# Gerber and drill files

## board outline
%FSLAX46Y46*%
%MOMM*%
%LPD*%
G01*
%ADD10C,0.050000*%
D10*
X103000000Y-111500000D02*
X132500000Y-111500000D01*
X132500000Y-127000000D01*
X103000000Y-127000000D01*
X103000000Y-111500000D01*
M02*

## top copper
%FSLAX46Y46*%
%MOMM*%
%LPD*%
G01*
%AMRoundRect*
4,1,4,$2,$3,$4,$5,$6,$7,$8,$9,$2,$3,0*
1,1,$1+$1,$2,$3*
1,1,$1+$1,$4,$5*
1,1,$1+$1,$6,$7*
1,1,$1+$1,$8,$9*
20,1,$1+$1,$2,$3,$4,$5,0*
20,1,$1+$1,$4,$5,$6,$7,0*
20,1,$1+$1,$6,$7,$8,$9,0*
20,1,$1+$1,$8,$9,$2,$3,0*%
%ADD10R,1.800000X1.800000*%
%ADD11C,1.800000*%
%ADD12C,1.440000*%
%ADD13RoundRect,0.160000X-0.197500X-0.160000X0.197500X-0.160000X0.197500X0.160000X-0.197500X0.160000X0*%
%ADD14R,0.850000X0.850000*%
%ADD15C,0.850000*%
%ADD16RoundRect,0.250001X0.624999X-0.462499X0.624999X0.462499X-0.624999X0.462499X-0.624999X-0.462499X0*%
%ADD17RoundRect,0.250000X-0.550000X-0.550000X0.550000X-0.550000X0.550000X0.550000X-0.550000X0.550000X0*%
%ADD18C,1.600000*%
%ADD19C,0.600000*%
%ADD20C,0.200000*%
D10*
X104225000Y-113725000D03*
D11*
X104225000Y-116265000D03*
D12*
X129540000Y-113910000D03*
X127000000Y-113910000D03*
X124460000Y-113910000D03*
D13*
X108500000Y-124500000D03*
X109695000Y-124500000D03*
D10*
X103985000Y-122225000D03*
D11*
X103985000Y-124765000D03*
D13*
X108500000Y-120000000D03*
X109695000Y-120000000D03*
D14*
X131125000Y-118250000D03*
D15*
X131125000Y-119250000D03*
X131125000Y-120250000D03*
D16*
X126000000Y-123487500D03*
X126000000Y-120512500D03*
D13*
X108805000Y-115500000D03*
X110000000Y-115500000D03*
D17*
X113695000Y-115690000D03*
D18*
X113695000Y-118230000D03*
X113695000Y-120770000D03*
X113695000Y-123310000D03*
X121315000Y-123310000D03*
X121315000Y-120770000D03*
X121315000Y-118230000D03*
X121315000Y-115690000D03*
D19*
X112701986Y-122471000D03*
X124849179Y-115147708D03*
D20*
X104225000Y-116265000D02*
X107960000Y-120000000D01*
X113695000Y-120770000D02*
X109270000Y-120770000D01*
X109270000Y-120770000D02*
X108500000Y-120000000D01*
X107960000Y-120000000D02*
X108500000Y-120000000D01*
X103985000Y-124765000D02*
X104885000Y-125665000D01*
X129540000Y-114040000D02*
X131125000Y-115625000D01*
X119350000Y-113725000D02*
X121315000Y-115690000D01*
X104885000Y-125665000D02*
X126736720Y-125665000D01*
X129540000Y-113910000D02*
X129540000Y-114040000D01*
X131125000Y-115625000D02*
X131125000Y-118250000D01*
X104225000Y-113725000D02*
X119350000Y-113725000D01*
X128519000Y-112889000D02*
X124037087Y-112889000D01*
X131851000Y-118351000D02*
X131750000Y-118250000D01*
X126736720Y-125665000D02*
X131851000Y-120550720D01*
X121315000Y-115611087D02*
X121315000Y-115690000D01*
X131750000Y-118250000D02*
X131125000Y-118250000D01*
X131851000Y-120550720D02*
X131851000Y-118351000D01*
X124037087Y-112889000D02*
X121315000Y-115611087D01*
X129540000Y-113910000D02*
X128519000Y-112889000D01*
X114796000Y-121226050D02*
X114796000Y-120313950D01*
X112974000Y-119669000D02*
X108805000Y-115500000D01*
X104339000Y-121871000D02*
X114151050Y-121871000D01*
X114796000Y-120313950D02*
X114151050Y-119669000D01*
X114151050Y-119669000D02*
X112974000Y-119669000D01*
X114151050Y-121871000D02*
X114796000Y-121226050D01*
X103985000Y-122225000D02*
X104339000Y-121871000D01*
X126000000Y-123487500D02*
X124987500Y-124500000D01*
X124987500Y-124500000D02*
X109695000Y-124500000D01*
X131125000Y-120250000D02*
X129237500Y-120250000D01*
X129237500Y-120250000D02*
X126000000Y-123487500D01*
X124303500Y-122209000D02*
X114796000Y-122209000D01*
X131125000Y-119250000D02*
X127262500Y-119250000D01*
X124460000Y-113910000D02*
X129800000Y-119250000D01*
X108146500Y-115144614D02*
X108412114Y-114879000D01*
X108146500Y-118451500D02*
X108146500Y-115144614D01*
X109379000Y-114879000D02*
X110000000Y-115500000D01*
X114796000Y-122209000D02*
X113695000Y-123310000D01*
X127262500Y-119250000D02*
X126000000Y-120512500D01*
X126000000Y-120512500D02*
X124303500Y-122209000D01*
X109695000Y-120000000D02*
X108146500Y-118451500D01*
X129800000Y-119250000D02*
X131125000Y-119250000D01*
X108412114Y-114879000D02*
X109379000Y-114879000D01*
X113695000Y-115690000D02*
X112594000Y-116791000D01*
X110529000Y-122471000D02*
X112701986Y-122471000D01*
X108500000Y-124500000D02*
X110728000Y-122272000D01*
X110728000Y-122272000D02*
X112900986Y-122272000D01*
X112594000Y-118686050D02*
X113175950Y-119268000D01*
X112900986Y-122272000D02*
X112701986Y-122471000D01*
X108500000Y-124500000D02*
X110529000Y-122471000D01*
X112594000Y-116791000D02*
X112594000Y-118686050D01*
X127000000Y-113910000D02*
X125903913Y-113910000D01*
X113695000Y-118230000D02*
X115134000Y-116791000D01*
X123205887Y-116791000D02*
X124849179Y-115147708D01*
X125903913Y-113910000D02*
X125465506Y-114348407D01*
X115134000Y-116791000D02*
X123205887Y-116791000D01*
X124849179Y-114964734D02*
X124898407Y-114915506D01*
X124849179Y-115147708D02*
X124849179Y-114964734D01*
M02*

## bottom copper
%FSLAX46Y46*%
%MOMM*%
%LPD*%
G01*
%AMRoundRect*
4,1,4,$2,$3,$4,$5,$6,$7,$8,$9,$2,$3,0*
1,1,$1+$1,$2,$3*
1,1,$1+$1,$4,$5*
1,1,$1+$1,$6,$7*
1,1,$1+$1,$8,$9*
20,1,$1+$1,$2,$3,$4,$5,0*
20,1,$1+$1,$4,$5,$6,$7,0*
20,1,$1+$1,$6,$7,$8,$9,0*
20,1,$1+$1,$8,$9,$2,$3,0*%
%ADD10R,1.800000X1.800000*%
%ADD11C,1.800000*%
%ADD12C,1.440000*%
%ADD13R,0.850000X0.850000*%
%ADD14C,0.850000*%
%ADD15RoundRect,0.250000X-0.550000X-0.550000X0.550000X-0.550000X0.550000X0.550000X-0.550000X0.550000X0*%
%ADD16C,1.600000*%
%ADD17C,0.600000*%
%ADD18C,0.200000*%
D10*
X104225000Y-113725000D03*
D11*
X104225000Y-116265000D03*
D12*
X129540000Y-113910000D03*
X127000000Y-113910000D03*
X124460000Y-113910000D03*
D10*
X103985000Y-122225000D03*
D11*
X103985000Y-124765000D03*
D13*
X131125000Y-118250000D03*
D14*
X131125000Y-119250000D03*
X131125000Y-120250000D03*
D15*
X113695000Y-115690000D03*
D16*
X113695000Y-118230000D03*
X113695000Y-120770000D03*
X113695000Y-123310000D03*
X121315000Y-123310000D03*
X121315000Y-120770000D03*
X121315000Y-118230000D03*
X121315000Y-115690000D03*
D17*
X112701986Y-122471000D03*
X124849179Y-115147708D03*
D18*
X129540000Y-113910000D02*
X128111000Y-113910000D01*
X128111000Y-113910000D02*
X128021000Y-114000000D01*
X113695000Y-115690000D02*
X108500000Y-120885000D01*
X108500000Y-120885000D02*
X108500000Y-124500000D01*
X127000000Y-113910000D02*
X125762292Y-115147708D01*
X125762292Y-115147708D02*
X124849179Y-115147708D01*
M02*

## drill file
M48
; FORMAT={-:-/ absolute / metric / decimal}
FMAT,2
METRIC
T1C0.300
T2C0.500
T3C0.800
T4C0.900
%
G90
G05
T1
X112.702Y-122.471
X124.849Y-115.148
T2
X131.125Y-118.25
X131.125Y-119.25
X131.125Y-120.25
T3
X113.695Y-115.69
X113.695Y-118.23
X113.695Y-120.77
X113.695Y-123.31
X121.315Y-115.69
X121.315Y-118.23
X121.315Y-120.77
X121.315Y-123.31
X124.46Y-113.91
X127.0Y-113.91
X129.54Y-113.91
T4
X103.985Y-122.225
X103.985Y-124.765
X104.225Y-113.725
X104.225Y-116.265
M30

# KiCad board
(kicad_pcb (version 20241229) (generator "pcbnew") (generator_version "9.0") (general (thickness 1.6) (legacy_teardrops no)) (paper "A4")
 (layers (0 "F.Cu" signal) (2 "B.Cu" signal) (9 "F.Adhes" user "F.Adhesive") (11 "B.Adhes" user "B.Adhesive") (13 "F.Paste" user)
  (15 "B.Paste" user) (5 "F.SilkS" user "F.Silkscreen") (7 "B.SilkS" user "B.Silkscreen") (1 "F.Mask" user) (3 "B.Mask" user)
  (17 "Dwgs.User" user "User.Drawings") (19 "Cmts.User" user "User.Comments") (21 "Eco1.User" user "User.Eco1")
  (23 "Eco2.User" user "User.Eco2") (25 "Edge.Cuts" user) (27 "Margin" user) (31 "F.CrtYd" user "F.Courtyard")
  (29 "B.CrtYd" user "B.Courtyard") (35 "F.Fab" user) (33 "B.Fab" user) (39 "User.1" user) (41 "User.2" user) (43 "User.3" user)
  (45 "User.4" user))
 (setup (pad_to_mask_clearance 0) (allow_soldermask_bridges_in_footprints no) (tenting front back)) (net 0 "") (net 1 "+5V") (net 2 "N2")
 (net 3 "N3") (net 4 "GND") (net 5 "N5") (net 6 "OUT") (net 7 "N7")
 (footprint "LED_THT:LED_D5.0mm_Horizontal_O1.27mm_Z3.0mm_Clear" (layer "F.Cu") (at 104.225 113.725 -90)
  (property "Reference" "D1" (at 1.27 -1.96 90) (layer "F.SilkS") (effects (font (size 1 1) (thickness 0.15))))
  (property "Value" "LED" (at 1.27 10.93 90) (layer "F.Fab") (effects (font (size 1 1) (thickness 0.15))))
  (pad "1" thru_hole rect (at 0 0 270) (size 1.8 1.8) (drill 0.9) (layers "*.Cu" "*.Mask") (remove_unused_layers no) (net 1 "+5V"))
  (pad "2" thru_hole circle (at 2.54 0 270) (size 1.8 1.8) (drill 0.9) (layers "*.Cu" "*.Mask") (remove_unused_layers no) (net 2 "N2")))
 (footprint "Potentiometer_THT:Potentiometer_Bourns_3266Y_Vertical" (layer "F.Cu") (at 129.54 113.91)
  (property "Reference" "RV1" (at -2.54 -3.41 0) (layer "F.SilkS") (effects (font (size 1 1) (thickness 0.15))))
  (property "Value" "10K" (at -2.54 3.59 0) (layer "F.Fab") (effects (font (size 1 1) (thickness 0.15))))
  (pad "1" thru_hole circle (at 0 0) (size 1.44 1.44) (drill 0.8) (layers "*.Cu" "*.Mask") (remove_unused_layers no) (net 1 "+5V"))
  (pad "2" thru_hole circle (at -2.54 0) (size 1.44 1.44) (drill 0.8) (layers "*.Cu" "*.Mask") (remove_unused_layers no) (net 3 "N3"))
  (pad "3" thru_hole circle (at -5.08 0) (size 1.44 1.44) (drill 0.8) (layers "*.Cu" "*.Mask") (remove_unused_layers no) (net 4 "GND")))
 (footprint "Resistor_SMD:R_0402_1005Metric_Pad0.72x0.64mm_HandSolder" (layer "F.Cu") (at 109.0975 124.5)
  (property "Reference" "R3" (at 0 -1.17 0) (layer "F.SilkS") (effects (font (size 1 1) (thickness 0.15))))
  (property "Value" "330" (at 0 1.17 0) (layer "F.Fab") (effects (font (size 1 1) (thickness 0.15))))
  (pad "1" smd roundrect (at -0.5975 0) (size 0.715 0.64) (layers "F.Cu" "F.Mask" "F.Paste") (roundrect_rratio 0.25) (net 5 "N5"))
  (pad "2" smd roundrect (at 0.5975 0) (size 0.715 0.64) (layers "F.Cu" "F.Mask" "F.Paste") (roundrect_rratio 0.25) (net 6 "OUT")))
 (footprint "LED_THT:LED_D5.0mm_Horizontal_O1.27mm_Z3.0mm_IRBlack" (layer "F.Cu") (at 103.985 122.225 -90)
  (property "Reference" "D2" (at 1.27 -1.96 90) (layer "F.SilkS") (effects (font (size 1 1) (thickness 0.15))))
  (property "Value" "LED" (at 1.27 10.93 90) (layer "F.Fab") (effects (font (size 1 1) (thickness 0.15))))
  (pad "1" thru_hole rect (at 0 0 270) (size 1.8 1.8) (drill 0.9) (layers "*.Cu" "*.Mask") (remove_unused_layers no) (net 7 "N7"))
  (pad "2" thru_hole circle (at 2.54 0 270) (size 1.8 1.8) (drill 0.9) (layers "*.Cu" "*.Mask") (remove_unused_layers no) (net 1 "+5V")))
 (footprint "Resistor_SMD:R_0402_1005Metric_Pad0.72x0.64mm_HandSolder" (layer "F.Cu") (at 109.0975 120)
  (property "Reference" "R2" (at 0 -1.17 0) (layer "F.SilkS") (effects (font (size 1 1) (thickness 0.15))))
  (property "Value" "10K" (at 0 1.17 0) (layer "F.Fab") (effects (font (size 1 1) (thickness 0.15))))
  (pad "1" smd roundrect (at -0.5975 0) (size 0.715 0.64) (layers "F.Cu" "F.Mask" "F.Paste") (roundrect_rratio 0.25) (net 2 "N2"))
  (pad "2" smd roundrect (at 0.5975 0) (size 0.715 0.64) (layers "F.Cu" "F.Mask" "F.Paste") (roundrect_rratio 0.25) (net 4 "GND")))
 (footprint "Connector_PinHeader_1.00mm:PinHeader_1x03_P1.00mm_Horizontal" (layer "F.Cu") (at 131.125 118.25)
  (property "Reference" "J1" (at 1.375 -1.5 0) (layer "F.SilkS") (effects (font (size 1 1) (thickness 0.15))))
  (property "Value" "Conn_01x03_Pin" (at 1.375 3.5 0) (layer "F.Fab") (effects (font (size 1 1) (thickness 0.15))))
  (pad "1" thru_hole rect (at 0 0) (size 0.85 0.85) (drill 0.5) (layers "*.Cu" "*.Mask") (remove_unused_layers no) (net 1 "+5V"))
  (pad "2" thru_hole circle (at 0 1) (size 0.85 0.85) (drill 0.5) (layers "*.Cu" "*.Mask") (remove_unused_layers no) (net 4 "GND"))
  (pad "3" thru_hole circle (at 0 2) (size 0.85 0.85) (drill 0.5) (layers "*.Cu" "*.Mask") (remove_unused_layers no) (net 6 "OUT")))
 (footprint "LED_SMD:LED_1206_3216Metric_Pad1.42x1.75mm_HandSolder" (layer "F.Cu") (at 126 122 90)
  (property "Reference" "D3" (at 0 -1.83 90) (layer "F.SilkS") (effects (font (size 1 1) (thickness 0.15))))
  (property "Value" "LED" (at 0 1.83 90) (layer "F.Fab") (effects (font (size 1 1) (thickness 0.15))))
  (pad "1" smd roundrect (at -1.4875 0 90) (size 1.425 1.75) (layers "F.Cu" "F.Mask" "F.Paste") (roundrect_rratio 0.175439) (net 6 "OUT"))
  (pad "2" smd roundrect (at 1.4875 0 90) (size 1.425 1.75) (layers "F.Cu" "F.Mask" "F.Paste") (roundrect_rratio 0.175439) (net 4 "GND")))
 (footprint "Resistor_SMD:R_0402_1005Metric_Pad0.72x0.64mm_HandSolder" (layer "F.Cu") (at 109.4025 115.5)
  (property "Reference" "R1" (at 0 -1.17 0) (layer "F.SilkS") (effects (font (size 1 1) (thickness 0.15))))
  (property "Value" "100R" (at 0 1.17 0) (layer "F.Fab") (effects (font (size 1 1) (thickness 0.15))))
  (pad "1" smd roundrect (at -0.5975 0) (size 0.715 0.64) (layers "F.Cu" "F.Mask" "F.Paste") (roundrect_rratio 0.25) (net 7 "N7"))
  (pad "2" smd roundrect (at 0.5975 0) (size 0.715 0.64) (layers "F.Cu" "F.Mask" "F.Paste") (roundrect_rratio 0.25) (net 4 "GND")))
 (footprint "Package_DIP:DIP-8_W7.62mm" (layer "F.Cu") (at 113.695 115.69)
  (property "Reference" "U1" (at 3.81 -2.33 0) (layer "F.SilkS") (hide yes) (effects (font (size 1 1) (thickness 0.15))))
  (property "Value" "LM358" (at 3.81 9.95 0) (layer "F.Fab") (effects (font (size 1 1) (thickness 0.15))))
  (pad "1" thru_hole roundrect (at 0 0) (size 1.6 1.6) (drill 0.8) (layers "*.Cu" "*.Mask") (remove_unused_layers no)
   (roundrect_rratio 0.15625) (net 5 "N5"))
  (pad "2" thru_hole circle (at 0 2.54) (size 1.6 1.6) (drill 0.8) (layers "*.Cu" "*.Mask") (remove_unused_layers no) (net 3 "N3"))
  (pad "3" thru_hole circle (at 0 5.08) (size 1.6 1.6) (drill 0.8) (layers "*.Cu" "*.Mask") (remove_unused_layers no) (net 2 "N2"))
  (pad "4" thru_hole circle (at 0 7.62) (size 1.6 1.6) (drill 0.8) (layers "*.Cu" "*.Mask") (remove_unused_layers no) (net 4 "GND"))
  (pad "5" thru_hole circle (at 7.62 7.62) (size 1.6 1.6) (drill 0.8) (layers "*.Cu" "*.Mask") (remove_unused_layers no))
  (pad "6" thru_hole circle (at 7.62 5.08) (size 1.6 1.6) (drill 0.8) (layers "*.Cu" "*.Mask") (remove_unused_layers no))
  (pad "7" thru_hole circle (at 7.62 2.54) (size 1.6 1.6) (drill 0.8) (layers "*.Cu" "*.Mask") (remove_unused_layers no))
  (pad "8" thru_hole circle (at 7.62 0) (size 1.6 1.6) (drill 0.8) (layers "*.Cu" "*.Mask") (remove_unused_layers no) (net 1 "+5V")))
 (gr_rect (start 103 111.5) (end 132.5 127) (stroke (width 0.05) (type default)) (fill no) (layer "Edge.Cuts"))
 (segment (start 104.225 116.265) (end 107.96 120) (width 0.2) (layer "F.Cu") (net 2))
 (segment (start 113.695 120.77) (end 109.27 120.77) (width 0.2) (layer "F.Cu") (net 2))
 (segment (start 109.27 120.77) (end 108.5 120) (width 0.2) (layer "F.Cu") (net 2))
 (segment (start 107.96 120) (end 108.5 120) (width 0.2) (layer "F.Cu") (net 2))
 (segment (start 103.985 124.765) (end 104.885 125.665) (width 0.2) (layer "F.Cu") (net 1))
 (segment (start 129.54 114.04) (end 131.125 115.625) (width 0.2) (layer "F.Cu") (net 1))
 (segment (start 119.35 113.725) (end 121.315 115.69) (width 0.2) (layer "F.Cu") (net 1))
 (segment (start 104.885 125.665) (end 126.73672 125.665) (width 0.2) (layer "F.Cu") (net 1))
 (segment (start 129.54 113.91) (end 129.54 114.04) (width 0.2) (layer "F.Cu") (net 1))
 (segment (start 131.125 115.625) (end 131.125 118.25) (width 0.2) (layer "F.Cu") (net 1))
 (segment (start 104.225 113.725) (end 119.35 113.725) (width 0.2) (layer "F.Cu") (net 1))
 (segment (start 128.519 112.889) (end 124.037087 112.889) (width 0.2) (layer "F.Cu") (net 1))
 (segment (start 131.851 118.351) (end 131.75 118.25) (width 0.2) (layer "F.Cu") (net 1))
 (segment (start 126.73672 125.665) (end 131.851 120.55072) (width 0.2) (layer "F.Cu") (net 1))
 (segment (start 121.315 115.611087) (end 121.315 115.69) (width 0.2) (layer "F.Cu") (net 1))
 (segment (start 131.75 118.25) (end 131.125 118.25) (width 0.2) (layer "F.Cu") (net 1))
 (segment (start 131.851 120.55072) (end 131.851 118.351) (width 0.2) (layer "F.Cu") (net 1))
 (segment (start 124.037087 112.889) (end 121.315 115.611087) (width 0.2) (layer "F.Cu") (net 1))
 (segment (start 129.54 113.91) (end 128.519 112.889) (width 0.2) (layer "F.Cu") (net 1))
 (segment (start 129.54 113.91) (end 128.111 113.91) (width 0.2) (layer "B.Cu") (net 1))
 (segment (start 128.111 113.91) (end 128.021 114) (width 0.2) (layer "B.Cu") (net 1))
 (segment (start 114.796 121.22605) (end 114.796 120.31395) (width 0.2) (layer "F.Cu") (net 7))
 (segment (start 112.974 119.669) (end 108.805 115.5) (width 0.2) (layer "F.Cu") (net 7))
 (segment (start 104.339 121.871) (end 114.15105 121.871) (width 0.2) (layer "F.Cu") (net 7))
 (segment (start 114.796 120.31395) (end 114.15105 119.669) (width 0.2) (layer "F.Cu") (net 7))
 (segment (start 114.15105 119.669) (end 112.974 119.669) (width 0.2) (layer "F.Cu") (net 7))
 (segment (start 114.15105 121.871) (end 114.796 121.22605) (width 0.2) (layer "F.Cu") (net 7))
 (segment (start 103.985 122.225) (end 104.339 121.871) (width 0.2) (layer "F.Cu") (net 7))
 (segment (start 126 123.4875) (end 124.9875 124.5) (width 0.2) (layer "F.Cu") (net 6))
 (segment (start 124.9875 124.5) (end 109.695 124.5) (width 0.2) (layer "F.Cu") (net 6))
 (segment (start 131.125 120.25) (end 129.2375 120.25) (width 0.2) (layer "F.Cu") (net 6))
 (segment (start 129.2375 120.25) (end 126 123.4875) (width 0.2) (layer "F.Cu") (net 6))
 (segment (start 124.3035 122.209) (end 114.796 122.209) (width 0.2) (layer "F.Cu") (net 4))
 (segment (start 131.125 119.25) (end 127.2625 119.25) (width 0.2) (layer "F.Cu") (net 4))
 (segment (start 124.46 113.91) (end 129.8 119.25) (width 0.2) (layer "F.Cu") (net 4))
 (segment (start 108.1465 115.144614) (end 108.412114 114.879) (width 0.2) (layer "F.Cu") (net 4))
 (segment (start 108.1465 118.4515) (end 108.1465 115.144614) (width 0.2) (layer "F.Cu") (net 4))
 (segment (start 109.379 114.879) (end 110 115.5) (width 0.2) (layer "F.Cu") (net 4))
 (segment (start 114.796 122.209) (end 113.695 123.31) (width 0.2) (layer "F.Cu") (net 4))
 (segment (start 127.2625 119.25) (end 126 120.5125) (width 0.2) (layer "F.Cu") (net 4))
 (segment (start 126 120.5125) (end 124.3035 122.209) (width 0.2) (layer "F.Cu") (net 4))
 (segment (start 109.695 120) (end 108.1465 118.4515) (width 0.2) (layer "F.Cu") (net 4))
 (segment (start 129.8 119.25) (end 131.125 119.25) (width 0.2) (layer "F.Cu") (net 4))
 (segment (start 108.412114 114.879) (end 109.379 114.879) (width 0.2) (layer "F.Cu") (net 4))
 (segment (start 113.695 115.69) (end 112.594 116.791) (width 0.2) (layer "F.Cu") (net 5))
 (segment (start 110.529 122.471) (end 112.701986 122.471) (width 0.2) (layer "F.Cu") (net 5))
 (segment (start 108.5 124.5) (end 110.728 122.272) (width 0.2) (layer "F.Cu") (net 5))
 (segment (start 110.728 122.272) (end 112.900986 122.272) (width 0.2) (layer "F.Cu") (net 5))
 (segment (start 112.594 118.68605) (end 113.17595 119.268) (width 0.2) (layer "F.Cu") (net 5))
 (segment (start 112.900986 122.272) (end 112.701986 122.471) (width 0.2) (layer "F.Cu") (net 5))
 (segment (start 108.5 124.5) (end 110.529 122.471) (width 0.2) (layer "F.Cu") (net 5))
 (segment (start 112.594 116.791) (end 112.594 118.68605) (width 0.2) (layer "F.Cu") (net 5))
 (via (at 112.701986 122.471) (size 0.6) (drill 0.3) (layers "F.Cu" "B.Cu") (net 5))
 (segment (start 113.695 115.69) (end 108.5 120.885) (width 0.2) (layer "B.Cu") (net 5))
 (segment (start 108.5 120.885) (end 108.5 124.5) (width 0.2) (layer "B.Cu") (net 5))
 (segment (start 127 113.91) (end 125.903913 113.91) (width 0.2) (layer "F.Cu") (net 3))
 (segment (start 113.695 118.23) (end 115.134 116.791) (width 0.2) (layer "F.Cu") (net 3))
 (segment (start 123.205887 116.791) (end 124.849179 115.147708) (width 0.2) (layer "F.Cu") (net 3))
 (segment (start 125.903913 113.91) (end 125.465506 114.348407) (width 0.2) (layer "F.Cu") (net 3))
 (segment (start 115.134 116.791) (end 123.205887 116.791) (width 0.2) (layer "F.Cu") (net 3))
 (segment (start 124.849179 114.964734) (end 124.898407 114.915506) (width 0.2) (layer "F.Cu") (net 3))
 (segment (start 124.849179 115.147708) (end 124.849179 114.964734) (width 0.2) (layer "F.Cu") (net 3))
 (via (at 124.849179 115.147708) (size 0.6) (drill 0.3) (layers "F.Cu" "B.Cu") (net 3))
 (segment (start 127 113.91) (end 125.762292 115.147708) (width 0.2) (layer "B.Cu") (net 3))
 (segment (start 125.762292 115.147708) (end 124.849179 115.147708) (width 0.2) (layer "B.Cu") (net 3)))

